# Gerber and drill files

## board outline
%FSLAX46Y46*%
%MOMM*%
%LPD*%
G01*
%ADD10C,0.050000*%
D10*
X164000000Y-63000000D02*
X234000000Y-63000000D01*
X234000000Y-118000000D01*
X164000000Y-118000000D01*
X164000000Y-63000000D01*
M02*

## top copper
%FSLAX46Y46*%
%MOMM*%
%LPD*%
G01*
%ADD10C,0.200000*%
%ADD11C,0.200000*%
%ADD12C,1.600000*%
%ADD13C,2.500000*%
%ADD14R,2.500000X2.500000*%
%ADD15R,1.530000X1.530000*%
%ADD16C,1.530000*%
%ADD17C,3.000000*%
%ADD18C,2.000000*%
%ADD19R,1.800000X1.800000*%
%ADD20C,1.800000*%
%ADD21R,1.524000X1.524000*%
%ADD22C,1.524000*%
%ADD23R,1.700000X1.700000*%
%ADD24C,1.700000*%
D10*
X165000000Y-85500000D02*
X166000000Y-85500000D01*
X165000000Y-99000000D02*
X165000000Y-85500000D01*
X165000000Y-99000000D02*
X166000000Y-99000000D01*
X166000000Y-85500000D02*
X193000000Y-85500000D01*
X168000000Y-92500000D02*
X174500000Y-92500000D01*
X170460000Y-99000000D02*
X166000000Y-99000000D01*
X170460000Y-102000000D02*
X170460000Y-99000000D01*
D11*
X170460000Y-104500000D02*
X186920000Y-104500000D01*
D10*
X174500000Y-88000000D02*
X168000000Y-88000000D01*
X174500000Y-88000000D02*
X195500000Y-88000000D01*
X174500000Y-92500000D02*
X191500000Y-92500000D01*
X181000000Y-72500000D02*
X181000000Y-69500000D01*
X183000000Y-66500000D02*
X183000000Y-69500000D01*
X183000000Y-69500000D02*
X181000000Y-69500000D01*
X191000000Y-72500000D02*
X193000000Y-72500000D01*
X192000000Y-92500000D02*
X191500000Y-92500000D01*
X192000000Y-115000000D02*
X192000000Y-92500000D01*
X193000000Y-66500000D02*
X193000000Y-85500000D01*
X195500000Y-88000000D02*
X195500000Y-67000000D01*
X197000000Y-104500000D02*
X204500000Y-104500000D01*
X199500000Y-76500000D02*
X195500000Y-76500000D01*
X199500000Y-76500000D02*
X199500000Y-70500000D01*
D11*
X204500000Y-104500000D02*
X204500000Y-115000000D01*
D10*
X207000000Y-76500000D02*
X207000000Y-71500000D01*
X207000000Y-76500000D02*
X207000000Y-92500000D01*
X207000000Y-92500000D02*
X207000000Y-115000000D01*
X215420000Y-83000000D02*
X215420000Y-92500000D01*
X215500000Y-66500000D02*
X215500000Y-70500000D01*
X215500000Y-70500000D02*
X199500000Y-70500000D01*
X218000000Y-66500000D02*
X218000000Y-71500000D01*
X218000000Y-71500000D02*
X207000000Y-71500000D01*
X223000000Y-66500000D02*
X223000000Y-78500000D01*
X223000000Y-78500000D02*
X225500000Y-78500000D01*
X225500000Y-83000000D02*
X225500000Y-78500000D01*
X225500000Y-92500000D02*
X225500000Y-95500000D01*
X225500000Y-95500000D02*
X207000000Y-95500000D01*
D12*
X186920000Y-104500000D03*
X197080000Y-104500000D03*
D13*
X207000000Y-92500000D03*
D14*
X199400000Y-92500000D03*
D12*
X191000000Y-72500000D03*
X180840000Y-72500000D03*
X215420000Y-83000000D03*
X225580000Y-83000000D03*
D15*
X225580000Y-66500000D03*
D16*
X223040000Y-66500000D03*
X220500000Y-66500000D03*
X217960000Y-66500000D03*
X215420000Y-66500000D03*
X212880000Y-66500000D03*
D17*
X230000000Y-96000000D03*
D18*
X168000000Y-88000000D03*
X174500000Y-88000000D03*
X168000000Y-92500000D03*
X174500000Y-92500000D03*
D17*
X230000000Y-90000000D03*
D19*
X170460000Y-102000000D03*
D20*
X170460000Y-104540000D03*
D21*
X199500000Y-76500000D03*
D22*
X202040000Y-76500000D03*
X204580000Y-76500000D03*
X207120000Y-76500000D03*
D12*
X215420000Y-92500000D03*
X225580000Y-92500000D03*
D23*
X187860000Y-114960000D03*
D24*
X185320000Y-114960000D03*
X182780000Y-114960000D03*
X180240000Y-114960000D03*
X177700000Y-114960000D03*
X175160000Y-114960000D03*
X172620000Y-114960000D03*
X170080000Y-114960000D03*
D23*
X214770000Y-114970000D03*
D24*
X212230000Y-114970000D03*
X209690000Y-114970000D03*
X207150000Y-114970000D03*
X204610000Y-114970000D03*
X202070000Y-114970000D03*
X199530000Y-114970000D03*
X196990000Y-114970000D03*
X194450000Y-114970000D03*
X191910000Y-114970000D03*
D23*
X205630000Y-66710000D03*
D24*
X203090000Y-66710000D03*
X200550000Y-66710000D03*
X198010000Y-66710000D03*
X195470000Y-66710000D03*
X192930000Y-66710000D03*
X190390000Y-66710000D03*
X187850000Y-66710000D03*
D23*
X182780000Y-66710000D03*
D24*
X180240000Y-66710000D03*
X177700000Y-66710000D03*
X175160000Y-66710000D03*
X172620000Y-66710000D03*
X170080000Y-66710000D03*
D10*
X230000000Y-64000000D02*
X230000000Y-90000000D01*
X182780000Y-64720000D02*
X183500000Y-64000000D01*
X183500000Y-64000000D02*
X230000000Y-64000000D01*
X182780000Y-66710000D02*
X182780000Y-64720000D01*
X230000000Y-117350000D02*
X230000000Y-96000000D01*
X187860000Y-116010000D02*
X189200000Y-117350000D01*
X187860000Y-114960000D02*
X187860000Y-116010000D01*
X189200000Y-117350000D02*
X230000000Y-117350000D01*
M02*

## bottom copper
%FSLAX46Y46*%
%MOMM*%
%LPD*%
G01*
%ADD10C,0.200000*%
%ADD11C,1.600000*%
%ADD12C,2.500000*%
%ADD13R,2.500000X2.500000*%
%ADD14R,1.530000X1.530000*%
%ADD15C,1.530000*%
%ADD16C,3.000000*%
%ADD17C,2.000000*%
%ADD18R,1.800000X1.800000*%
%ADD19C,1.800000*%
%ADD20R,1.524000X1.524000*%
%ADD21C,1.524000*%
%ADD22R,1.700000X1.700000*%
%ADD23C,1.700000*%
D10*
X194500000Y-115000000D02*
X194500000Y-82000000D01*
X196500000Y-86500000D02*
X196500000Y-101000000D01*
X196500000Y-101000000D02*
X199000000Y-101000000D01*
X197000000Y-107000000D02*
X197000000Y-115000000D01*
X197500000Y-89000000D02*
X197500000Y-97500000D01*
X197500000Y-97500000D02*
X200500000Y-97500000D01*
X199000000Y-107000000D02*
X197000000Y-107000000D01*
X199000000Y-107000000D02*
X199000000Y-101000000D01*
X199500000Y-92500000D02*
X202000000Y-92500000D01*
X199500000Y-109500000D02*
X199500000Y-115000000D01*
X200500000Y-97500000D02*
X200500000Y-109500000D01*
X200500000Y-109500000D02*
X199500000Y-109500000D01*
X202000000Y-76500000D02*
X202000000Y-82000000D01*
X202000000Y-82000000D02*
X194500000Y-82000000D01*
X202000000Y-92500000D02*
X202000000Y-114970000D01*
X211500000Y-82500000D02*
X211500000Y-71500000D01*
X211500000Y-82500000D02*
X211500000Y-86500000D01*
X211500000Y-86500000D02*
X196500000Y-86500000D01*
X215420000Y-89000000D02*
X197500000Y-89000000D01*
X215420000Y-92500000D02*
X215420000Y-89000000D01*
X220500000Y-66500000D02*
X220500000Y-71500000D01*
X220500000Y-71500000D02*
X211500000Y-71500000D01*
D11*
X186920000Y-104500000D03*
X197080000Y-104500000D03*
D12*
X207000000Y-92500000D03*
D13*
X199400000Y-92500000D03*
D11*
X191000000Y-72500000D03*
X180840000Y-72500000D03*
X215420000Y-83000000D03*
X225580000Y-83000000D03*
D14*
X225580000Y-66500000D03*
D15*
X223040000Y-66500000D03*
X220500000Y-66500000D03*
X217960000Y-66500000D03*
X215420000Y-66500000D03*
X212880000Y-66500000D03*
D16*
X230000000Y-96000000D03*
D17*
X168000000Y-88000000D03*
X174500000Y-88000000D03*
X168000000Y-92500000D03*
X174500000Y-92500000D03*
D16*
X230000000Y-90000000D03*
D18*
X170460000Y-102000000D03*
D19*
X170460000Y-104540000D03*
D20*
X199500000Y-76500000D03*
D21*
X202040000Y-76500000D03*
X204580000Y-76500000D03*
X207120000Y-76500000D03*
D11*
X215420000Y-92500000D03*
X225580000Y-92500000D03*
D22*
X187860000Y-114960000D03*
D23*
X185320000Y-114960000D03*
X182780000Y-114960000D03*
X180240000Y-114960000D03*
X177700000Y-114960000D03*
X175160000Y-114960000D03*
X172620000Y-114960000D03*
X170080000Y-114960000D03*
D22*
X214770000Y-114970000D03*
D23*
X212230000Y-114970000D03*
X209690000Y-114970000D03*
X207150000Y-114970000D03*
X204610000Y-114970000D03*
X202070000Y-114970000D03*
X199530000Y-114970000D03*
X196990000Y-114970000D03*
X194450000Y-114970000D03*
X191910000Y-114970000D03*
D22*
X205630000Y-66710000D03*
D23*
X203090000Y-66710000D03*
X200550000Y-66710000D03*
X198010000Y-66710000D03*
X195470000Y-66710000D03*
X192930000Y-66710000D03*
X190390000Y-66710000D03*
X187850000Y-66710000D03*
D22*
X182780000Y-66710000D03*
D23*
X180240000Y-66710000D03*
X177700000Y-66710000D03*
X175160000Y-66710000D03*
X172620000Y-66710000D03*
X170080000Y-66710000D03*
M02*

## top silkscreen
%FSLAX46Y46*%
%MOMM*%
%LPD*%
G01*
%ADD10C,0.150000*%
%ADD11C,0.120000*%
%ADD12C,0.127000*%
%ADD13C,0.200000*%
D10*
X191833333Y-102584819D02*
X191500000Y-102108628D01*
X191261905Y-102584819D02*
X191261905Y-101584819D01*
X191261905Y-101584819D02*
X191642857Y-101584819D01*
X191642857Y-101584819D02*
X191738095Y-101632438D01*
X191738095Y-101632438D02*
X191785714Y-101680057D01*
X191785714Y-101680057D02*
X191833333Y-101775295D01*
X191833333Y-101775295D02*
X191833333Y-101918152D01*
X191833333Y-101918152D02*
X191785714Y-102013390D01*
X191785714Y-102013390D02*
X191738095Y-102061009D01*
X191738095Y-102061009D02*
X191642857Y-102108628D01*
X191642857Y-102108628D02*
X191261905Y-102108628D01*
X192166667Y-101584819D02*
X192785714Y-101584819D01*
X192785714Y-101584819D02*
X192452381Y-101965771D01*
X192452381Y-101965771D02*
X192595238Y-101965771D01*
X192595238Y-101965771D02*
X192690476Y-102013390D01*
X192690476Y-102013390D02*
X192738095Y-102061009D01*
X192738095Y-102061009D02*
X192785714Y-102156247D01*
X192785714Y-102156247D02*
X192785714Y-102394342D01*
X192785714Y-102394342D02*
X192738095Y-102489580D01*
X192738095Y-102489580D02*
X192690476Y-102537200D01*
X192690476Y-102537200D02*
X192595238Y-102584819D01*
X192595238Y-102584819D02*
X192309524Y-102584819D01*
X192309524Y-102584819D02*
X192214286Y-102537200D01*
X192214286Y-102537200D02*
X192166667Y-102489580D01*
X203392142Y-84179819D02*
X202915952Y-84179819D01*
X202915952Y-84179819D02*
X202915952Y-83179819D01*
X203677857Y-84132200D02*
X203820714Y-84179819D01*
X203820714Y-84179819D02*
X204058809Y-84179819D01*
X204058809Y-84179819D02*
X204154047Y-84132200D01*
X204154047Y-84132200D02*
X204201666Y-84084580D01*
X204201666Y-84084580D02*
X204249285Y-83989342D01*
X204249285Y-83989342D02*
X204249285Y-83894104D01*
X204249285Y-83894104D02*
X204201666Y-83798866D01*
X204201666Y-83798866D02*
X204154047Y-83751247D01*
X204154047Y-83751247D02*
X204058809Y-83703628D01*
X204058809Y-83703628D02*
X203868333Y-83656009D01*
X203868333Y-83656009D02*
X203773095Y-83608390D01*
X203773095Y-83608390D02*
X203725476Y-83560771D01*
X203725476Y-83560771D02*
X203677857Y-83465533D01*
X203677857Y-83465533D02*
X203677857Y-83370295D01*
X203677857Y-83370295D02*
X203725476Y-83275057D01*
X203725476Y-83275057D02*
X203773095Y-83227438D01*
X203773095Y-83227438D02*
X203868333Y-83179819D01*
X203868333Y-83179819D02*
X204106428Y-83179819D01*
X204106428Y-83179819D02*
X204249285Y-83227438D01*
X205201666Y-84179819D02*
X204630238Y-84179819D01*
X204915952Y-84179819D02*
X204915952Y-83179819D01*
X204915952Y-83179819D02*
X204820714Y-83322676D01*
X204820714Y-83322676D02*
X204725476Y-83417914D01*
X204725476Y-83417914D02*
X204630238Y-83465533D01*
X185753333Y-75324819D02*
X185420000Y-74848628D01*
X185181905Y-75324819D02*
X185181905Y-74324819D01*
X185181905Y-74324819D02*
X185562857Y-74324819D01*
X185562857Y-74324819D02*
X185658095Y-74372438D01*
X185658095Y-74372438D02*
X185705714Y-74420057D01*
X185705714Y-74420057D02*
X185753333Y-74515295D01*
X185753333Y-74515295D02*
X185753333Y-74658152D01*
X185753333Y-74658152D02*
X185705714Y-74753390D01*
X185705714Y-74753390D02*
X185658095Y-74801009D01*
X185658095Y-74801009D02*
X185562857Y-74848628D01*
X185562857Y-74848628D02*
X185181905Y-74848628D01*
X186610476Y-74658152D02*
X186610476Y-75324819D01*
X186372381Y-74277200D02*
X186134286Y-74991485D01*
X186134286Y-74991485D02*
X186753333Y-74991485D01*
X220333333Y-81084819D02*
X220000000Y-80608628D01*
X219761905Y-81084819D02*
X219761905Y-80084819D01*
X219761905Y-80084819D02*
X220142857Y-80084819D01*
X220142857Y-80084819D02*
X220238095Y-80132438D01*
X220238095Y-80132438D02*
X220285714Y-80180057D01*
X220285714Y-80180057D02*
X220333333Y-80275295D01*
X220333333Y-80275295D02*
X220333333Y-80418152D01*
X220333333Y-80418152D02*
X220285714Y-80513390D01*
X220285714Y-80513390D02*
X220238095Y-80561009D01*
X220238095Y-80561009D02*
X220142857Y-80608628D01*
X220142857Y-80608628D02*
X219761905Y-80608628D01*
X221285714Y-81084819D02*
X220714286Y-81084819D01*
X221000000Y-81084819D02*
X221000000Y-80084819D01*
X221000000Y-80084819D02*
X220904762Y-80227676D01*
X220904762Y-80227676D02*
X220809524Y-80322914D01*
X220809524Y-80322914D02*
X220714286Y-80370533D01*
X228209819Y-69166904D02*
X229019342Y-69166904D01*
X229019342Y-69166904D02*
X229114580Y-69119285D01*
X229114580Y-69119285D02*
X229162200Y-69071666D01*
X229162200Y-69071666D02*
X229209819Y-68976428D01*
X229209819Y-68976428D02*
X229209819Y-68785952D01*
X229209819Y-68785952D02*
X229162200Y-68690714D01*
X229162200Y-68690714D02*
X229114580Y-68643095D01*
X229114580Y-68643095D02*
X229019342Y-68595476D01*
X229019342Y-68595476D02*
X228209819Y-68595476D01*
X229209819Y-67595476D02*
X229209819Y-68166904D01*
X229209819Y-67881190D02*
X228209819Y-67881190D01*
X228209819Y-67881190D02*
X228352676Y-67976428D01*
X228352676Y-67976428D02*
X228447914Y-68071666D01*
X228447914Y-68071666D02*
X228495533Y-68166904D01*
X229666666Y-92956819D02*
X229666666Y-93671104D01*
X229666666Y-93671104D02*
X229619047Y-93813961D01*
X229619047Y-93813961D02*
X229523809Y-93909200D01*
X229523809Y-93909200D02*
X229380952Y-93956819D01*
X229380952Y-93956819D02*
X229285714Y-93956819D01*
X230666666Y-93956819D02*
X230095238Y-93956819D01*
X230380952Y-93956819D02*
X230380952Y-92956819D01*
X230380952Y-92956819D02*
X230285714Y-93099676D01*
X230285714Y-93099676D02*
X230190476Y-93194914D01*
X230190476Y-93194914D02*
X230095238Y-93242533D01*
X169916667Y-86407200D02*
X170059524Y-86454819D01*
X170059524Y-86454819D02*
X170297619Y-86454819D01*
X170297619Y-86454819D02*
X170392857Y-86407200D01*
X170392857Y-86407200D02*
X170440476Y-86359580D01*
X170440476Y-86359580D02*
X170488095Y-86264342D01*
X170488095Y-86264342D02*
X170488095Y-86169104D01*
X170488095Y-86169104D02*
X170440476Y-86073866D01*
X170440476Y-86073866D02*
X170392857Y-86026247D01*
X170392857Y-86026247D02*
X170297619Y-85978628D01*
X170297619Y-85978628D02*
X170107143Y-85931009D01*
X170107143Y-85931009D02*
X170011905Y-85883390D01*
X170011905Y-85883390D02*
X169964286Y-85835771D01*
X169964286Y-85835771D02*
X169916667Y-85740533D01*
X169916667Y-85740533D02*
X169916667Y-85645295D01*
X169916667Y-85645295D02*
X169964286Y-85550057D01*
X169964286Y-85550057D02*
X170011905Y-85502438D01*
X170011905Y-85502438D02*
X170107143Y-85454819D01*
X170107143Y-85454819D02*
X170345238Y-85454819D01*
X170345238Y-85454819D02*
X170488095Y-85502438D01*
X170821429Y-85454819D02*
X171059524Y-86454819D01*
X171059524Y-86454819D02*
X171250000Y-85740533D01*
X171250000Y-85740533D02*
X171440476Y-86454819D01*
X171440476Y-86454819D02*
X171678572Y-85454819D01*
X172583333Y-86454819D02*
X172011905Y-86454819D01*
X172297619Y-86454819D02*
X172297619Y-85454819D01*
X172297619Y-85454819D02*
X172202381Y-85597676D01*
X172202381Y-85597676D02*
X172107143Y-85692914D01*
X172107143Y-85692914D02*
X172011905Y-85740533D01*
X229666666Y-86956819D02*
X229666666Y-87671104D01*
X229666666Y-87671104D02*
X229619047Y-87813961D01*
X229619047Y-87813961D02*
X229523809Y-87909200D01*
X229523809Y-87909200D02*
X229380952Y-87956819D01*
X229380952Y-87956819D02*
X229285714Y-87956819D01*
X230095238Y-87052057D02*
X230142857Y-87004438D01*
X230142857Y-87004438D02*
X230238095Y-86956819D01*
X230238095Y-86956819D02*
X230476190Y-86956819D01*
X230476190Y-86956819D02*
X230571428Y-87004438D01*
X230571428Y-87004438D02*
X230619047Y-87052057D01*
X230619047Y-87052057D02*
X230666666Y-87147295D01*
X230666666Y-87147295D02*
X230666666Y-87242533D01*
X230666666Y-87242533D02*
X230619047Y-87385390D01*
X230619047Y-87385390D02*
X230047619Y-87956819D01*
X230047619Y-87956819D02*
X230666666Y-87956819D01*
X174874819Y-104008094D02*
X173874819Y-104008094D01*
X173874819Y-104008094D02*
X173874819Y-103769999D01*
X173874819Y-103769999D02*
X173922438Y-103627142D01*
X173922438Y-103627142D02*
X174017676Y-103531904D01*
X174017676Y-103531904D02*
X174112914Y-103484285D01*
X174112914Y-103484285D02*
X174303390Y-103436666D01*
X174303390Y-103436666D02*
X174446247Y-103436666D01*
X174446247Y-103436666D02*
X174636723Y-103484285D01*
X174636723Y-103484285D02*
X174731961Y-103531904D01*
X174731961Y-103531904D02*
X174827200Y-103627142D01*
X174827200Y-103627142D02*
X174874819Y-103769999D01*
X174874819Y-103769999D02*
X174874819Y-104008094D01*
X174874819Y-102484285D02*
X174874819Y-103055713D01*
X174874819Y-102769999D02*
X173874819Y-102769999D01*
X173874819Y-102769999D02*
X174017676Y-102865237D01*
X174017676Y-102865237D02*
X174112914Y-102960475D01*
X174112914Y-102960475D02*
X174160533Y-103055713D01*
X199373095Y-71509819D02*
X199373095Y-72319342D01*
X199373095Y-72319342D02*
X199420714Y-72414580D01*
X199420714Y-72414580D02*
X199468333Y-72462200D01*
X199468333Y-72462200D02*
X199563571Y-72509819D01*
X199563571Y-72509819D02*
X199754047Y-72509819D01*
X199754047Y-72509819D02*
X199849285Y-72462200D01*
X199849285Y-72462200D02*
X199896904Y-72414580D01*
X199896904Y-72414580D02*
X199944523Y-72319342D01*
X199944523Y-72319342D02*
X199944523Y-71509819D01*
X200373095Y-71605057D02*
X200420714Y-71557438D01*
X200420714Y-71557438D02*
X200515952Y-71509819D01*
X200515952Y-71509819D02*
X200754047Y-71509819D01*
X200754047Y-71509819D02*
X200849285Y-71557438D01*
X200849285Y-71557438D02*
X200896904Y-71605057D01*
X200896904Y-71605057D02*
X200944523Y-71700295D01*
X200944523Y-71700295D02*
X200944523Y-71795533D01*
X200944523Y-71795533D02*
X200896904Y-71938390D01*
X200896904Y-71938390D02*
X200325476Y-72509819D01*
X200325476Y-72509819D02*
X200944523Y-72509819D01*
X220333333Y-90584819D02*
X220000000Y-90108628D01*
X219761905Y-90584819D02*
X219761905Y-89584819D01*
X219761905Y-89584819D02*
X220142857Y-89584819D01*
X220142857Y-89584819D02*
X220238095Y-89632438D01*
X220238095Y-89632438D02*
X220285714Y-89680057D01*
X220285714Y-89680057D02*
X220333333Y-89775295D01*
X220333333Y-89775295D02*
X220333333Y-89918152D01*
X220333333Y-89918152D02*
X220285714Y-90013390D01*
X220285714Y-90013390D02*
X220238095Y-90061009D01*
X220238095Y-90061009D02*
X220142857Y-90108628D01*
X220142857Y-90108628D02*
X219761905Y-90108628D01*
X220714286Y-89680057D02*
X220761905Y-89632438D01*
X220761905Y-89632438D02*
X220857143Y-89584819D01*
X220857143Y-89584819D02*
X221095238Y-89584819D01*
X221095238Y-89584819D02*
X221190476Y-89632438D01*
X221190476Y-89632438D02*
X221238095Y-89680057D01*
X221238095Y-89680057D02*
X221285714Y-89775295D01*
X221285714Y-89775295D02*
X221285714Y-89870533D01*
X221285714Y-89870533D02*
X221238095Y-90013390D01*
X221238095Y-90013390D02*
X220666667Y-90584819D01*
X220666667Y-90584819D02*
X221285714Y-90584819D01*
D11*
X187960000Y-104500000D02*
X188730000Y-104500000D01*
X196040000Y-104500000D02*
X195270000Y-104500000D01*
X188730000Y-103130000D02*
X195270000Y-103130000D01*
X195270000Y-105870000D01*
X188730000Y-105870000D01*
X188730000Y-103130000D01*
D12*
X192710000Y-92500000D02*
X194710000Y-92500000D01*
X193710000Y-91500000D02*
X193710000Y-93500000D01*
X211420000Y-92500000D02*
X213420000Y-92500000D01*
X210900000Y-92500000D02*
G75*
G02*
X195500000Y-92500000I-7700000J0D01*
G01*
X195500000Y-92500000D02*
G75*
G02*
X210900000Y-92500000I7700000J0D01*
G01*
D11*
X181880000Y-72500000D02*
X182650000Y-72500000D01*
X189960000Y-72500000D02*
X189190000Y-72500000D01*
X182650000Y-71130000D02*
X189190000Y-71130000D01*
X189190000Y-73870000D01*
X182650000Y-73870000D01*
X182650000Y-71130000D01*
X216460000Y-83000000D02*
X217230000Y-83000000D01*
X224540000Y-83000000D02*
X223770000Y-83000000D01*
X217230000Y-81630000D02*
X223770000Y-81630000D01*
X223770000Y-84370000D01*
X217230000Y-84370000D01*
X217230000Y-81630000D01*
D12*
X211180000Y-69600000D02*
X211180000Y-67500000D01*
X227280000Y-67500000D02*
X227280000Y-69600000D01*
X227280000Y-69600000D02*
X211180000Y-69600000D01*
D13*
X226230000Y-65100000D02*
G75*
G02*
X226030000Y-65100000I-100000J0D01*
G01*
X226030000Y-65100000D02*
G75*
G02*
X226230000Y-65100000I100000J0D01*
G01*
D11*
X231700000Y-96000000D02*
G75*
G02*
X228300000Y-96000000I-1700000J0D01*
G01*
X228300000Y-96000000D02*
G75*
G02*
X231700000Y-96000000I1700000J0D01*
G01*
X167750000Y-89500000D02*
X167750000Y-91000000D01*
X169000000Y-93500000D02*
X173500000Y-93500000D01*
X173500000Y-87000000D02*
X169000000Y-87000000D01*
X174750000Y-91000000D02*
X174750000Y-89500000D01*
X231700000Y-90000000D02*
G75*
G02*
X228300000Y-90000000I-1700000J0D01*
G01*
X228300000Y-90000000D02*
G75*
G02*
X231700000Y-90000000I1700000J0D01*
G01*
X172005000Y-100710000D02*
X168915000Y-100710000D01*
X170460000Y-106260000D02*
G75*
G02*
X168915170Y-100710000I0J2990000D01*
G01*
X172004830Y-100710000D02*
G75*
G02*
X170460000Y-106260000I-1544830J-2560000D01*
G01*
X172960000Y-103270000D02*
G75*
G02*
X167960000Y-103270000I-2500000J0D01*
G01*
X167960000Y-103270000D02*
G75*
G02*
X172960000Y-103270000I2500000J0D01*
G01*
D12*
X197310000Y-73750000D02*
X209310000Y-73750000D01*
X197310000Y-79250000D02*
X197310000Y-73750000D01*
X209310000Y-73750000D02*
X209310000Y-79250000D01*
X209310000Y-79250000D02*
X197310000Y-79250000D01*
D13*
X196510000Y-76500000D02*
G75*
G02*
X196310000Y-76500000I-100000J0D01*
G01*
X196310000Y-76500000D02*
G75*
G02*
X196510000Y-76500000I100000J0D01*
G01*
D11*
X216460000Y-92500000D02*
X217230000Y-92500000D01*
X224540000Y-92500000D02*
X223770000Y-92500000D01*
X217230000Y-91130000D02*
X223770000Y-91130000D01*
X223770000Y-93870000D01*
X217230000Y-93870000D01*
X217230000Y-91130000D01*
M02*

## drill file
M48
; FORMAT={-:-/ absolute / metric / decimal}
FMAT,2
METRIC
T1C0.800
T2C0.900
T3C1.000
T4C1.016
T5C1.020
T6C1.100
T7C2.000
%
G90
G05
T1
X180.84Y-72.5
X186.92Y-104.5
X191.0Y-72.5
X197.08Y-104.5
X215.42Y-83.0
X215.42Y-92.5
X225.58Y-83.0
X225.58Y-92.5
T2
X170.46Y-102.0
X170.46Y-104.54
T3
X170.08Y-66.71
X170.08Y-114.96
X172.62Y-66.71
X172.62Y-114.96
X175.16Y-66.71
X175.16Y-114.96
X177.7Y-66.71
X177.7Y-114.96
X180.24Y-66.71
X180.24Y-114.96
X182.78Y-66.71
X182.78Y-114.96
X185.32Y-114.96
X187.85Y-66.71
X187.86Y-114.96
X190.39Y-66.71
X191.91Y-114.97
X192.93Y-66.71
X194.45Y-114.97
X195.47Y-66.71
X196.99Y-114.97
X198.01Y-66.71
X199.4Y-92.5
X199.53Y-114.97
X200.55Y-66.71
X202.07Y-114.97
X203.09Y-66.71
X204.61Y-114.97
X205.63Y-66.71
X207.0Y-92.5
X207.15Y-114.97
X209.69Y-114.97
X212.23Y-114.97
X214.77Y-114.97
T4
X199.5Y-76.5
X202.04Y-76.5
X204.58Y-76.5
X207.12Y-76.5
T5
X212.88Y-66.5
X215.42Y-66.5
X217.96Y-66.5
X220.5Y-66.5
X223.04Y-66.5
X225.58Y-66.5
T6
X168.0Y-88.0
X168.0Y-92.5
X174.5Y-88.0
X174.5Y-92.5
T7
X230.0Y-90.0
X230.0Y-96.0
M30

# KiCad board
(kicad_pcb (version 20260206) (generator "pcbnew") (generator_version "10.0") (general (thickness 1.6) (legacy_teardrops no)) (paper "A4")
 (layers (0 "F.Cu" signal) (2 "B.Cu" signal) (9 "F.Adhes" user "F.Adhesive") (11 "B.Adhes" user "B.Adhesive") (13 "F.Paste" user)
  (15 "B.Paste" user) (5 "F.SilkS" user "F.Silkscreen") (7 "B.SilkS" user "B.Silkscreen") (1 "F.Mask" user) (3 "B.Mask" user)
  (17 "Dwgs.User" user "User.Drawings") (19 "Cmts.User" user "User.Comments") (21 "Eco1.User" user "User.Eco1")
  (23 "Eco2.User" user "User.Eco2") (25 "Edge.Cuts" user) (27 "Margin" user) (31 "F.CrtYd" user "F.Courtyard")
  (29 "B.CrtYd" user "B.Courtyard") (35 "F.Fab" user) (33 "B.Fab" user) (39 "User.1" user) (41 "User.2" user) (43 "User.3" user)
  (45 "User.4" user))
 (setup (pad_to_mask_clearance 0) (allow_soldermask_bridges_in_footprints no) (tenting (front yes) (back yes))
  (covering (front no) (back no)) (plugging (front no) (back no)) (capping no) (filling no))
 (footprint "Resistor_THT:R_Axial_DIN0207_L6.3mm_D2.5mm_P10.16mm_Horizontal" (layer "F.Cu") (at 186.92 104.5)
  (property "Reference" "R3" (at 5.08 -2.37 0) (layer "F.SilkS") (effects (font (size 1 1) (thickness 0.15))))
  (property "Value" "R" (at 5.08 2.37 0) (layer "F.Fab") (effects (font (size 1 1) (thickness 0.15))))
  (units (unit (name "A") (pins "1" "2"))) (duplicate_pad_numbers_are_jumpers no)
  (fp_line (start 1.04 0) (end 1.81 0) (stroke (width 0.12) (type solid)) (layer "F.SilkS"))
  (fp_line (start 9.12 0) (end 8.35 0) (stroke (width 0.12) (type solid)) (layer "F.SilkS"))
  (fp_rect (start 1.81 -1.37) (end 8.35 1.37) (stroke (width 0.12) (type solid)) (fill no) (layer "F.SilkS"))
  (pad "1" thru_hole circle (at 0 0) (size 1.6 1.6) (drill 0.8) (layers "*.Cu" "*.Mask") (remove_unused_layers no) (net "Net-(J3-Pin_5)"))
  (pad "2" thru_hole circle (at 10.16 0) (size 1.6 1.6) (drill 0.8) (layers "*.Cu" "*.Mask") (remove_unused_layers no) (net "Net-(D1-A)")))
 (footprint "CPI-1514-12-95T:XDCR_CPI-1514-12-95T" (layer "F.Cu") (at 203.2 92.5)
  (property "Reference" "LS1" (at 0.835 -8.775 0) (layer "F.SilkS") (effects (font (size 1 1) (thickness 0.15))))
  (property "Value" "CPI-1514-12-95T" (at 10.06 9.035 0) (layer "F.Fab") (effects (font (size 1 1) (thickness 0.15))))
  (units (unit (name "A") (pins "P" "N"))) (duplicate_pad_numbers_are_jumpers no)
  (fp_line (start -10.49 0) (end -8.49 0) (stroke (width 0.127) (type solid)) (layer "F.SilkS"))
  (fp_line (start -9.49 -1) (end -9.49 1) (stroke (width 0.127) (type solid)) (layer "F.SilkS"))
  (fp_line (start 8.22 0) (end 10.22 0) (stroke (width 0.127) (type solid)) (layer "F.SilkS"))
  (fp_circle (center 0 0) (end 7.7 0) (stroke (width 0.127) (type solid)) (fill no) (layer "F.SilkS"))
  (pad "N" thru_hole circle (at 3.8 0) (size 2.5 2.5) (drill 1) (layers "*.Cu" "*.Mask") (remove_unused_layers no) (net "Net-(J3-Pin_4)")
   (solder_mask_margin 0.102))
  (pad "P" thru_hole rect (at -3.8 0) (size 2.5 2.5) (drill 1) (layers "*.Cu" "*.Mask") (remove_unused_layers no) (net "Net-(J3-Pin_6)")
   (solder_mask_margin 0.102)))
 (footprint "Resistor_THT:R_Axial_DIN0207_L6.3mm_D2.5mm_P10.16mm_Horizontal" (layer "F.Cu") (at 191 72.5 180)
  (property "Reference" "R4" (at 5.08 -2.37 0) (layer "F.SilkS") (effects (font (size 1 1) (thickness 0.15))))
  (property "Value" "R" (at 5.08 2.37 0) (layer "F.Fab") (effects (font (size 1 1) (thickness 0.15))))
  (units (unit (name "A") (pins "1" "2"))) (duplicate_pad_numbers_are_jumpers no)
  (fp_line (start 9.12 0) (end 8.35 0) (stroke (width 0.12) (type solid)) (layer "F.SilkS"))
  (fp_line (start 1.04 0) (end 1.81 0) (stroke (width 0.12) (type solid)) (layer "F.SilkS"))
  (fp_rect (start 1.81 -1.37) (end 8.35 1.37) (stroke (width 0.12) (type solid)) (fill no) (layer "F.SilkS"))
  (pad "1" thru_hole circle (at 0 0 180) (size 1.6 1.6) (drill 0.8) (layers "*.Cu" "*.Mask") (remove_unused_layers no) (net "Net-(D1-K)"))
  (pad "2" thru_hole circle (at 10.16 0 180) (size 1.6 1.6) (drill 0.8) (layers "*.Cu" "*.Mask") (remove_unused_layers no)
   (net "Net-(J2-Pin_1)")))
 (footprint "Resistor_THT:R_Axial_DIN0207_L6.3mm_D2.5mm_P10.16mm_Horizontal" (layer "F.Cu") (at 215.42 83)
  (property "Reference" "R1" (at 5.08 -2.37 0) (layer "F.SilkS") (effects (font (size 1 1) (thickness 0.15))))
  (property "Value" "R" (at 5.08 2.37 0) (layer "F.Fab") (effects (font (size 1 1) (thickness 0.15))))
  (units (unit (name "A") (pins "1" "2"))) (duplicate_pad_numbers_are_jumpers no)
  (fp_line (start 1.04 0) (end 1.81 0) (stroke (width 0.12) (type solid)) (layer "F.SilkS"))
  (fp_line (start 9.12 0) (end 8.35 0) (stroke (width 0.12) (type solid)) (layer "F.SilkS"))
  (fp_rect (start 1.81 -1.37) (end 8.35 1.37) (stroke (width 0.12) (type solid)) (fill no) (layer "F.SilkS"))
  (pad "1" thru_hole circle (at 0 0) (size 1.6 1.6) (drill 0.8) (layers "*.Cu" "*.Mask") (remove_unused_layers no) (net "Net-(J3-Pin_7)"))
  (pad "2" thru_hole circle (at 10.16 0) (size 1.6 1.6) (drill 0.8) (layers "*.Cu" "*.Mask") (remove_unused_layers no) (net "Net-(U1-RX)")))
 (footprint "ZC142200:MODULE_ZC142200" (layer "F.Cu") (at 219.23 66.5 -90)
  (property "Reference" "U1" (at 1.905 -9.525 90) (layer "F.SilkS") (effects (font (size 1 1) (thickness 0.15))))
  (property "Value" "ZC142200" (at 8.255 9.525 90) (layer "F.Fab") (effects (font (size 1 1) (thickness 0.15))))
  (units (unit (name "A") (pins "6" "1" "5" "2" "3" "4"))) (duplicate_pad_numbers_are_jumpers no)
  (fp_line (start 3.1 8.05) (end 1 8.05) (stroke (width 0.127) (type solid)) (layer "F.SilkS"))
  (fp_line (start 1 -8.05) (end 3.1 -8.05) (stroke (width 0.127) (type solid)) (layer "F.SilkS"))
  (fp_line (start 3.1 -8.05) (end 3.1 8.05) (stroke (width 0.127) (type solid)) (layer "F.SilkS"))
  (fp_circle (center -1.4 -6.9) (end -1.3 -6.9) (stroke (width 0.2) (type solid)) (fill no) (layer "F.SilkS"))
  (pad "1" thru_hole rect (at 0 -6.35 270) (size 1.53 1.53) (drill 1.02) (layers "*.Cu" "*.Mask") (remove_unused_layers no)
   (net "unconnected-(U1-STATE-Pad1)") (solder_mask_margin 0.102))
  (pad "2" thru_hole circle (at 0 -3.81 270) (size 1.53 1.53) (drill 1.02) (layers "*.Cu" "*.Mask") (remove_unused_layers no)
   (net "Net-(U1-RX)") (solder_mask_margin 0.102))
  (pad "3" thru_hole circle (at 0 -1.27 270) (size 1.53 1.53) (drill 1.02) (layers "*.Cu" "*.Mask") (remove_unused_layers no)
   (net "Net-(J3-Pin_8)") (solder_mask_margin 0.102))
  (pad "4" thru_hole circle (at 0 1.27 270) (size 1.53 1.53) (drill 1.02) (layers "*.Cu" "*.Mask") (remove_unused_layers no)
   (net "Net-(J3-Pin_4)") (solder_mask_margin 0.102))
  (pad "5" thru_hole circle (at 0 3.81 270) (size 1.53 1.53) (drill 1.02) (layers "*.Cu" "*.Mask") (remove_unused_layers no)
   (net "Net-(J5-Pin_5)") (solder_mask_margin 0.102))
  (pad "6" thru_hole circle (at 0 6.35 270) (size 1.53 1.53) (drill 1.02) (layers "*.Cu" "*.Mask") (remove_unused_layers no)
   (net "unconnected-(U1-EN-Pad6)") (solder_mask_margin 0.102)))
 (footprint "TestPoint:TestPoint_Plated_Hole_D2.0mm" (layer "F.Cu") (at 230 96)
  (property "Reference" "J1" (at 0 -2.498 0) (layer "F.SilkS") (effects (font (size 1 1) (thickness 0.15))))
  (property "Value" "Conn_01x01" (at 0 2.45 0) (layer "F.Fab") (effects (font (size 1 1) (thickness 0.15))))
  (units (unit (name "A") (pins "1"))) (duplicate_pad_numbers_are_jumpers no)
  (fp_circle (center 0 0) (end 0 -1.7) (stroke (width 0.12) (type solid)) (fill no) (layer "F.SilkS"))
  (pad "1" thru_hole circle (at 0 0) (size 3 3) (drill 2) (layers "*.Cu" "*.Mask") (remove_unused_layers no) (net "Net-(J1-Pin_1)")))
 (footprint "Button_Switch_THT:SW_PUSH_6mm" (layer "F.Cu") (at 168 88)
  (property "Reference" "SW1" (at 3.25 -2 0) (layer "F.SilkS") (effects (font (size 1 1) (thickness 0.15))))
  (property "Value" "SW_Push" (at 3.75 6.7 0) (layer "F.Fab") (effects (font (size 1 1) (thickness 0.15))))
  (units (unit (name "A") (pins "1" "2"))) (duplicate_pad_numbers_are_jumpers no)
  (fp_line (start -0.25 1.5) (end -0.25 3) (stroke (width 0.12) (type solid)) (layer "F.SilkS"))
  (fp_line (start 1 5.5) (end 5.5 5.5) (stroke (width 0.12) (type solid)) (layer "F.SilkS"))
  (fp_line (start 5.5 -1) (end 1 -1) (stroke (width 0.12) (type solid)) (layer "F.SilkS"))
  (fp_line (start 6.75 3) (end 6.75 1.5) (stroke (width 0.12) (type solid)) (layer "F.SilkS"))
  (pad "1" thru_hole circle (at 0 0 90) (size 2 2) (drill 1.1) (layers "*.Cu" "*.Mask") (remove_unused_layers no) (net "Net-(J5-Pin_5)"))
  (pad "1" thru_hole circle (at 6.5 0 90) (size 2 2) (drill 1.1) (layers "*.Cu" "*.Mask") (remove_unused_layers no) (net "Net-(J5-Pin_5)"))
  (pad "2" thru_hole circle (at 0 4.5 90) (size 2 2) (drill 1.1) (layers "*.Cu" "*.Mask") (remove_unused_layers no) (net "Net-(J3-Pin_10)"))
  (pad "2" thru_hole circle (at 6.5 4.5 90) (size 2 2) (drill 1.1) (layers "*.Cu" "*.Mask") (remove_unused_layers no)
   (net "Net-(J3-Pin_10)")))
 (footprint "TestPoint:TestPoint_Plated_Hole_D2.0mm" (layer "F.Cu") (at 230 90)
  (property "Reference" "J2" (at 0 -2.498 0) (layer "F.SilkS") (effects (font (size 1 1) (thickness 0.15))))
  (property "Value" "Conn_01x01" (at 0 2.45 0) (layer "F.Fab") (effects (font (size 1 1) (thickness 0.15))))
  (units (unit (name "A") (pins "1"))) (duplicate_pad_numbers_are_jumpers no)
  (fp_circle (center 0 0) (end 0 -1.7) (stroke (width 0.12) (type solid)) (fill no) (layer "F.SilkS"))
  (pad "1" thru_hole circle (at 0 0) (size 3 3) (drill 2) (layers "*.Cu" "*.Mask") (remove_unused_layers no) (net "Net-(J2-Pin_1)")))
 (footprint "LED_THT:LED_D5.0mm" (layer "F.Cu") (at 170.46 102 -90)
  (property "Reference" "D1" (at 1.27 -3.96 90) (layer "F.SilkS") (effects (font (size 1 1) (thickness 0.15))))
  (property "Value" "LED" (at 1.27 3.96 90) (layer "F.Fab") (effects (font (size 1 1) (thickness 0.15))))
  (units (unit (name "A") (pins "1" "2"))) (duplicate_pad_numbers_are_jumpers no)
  (fp_line (start -1.29 -1.545) (end -1.29 1.545) (stroke (width 0.12) (type solid)) (layer "F.SilkS"))
  (fp_arc (start 4.26 0) (mid 2.071779 2.880495) (end -1.29 1.54483) (stroke (width 0.12) (type solid)) (layer "F.SilkS"))
  (fp_arc (start -1.29 -1.54483) (mid 2.071779 -2.880495) (end 4.26 0) (stroke (width 0.12) (type solid)) (layer "F.SilkS"))
  (fp_circle (center 1.27 0) (end 3.77 0) (stroke (width 0.12) (type solid)) (fill no) (layer "F.SilkS"))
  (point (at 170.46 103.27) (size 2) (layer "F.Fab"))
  (pad "1" thru_hole rect (at 0 0 270) (size 1.8 1.8) (drill 0.9) (layers "*.Cu" "*.Mask") (remove_unused_layers no) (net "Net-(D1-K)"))
  (pad "2" thru_hole circle (at 2.54 0 270) (size 1.8 1.8) (drill 0.9) (layers "*.Cu" "*.Mask") (remove_unused_layers no) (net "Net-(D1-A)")))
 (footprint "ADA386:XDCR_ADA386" (layer "F.Cu") (at 203.31 76.5)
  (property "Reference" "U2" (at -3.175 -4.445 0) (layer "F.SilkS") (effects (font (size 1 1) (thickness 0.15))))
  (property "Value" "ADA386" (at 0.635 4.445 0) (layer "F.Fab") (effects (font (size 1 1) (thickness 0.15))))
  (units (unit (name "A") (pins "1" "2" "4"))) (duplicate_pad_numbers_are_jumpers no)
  (fp_line (start -6 -2.75) (end 6 -2.75) (stroke (width 0.127) (type solid)) (layer "F.SilkS"))
  (fp_line (start -6 2.75) (end -6 -2.75) (stroke (width 0.127) (type solid)) (layer "F.SilkS"))
  (fp_line (start 6 -2.75) (end 6 2.75) (stroke (width 0.127) (type solid)) (layer "F.SilkS"))
  (fp_line (start 6 2.75) (end -6 2.75) (stroke (width 0.127) (type solid)) (layer "F.SilkS"))
  (fp_circle (center -6.9 0) (end -6.8 0) (stroke (width 0.2) (type solid)) (fill no) (layer "F.SilkS"))
  (pad "1" thru_hole rect (at -3.81 0) (size 1.524 1.524) (drill 1.016) (layers "*.Cu" "*.Mask") (remove_unused_layers no)
   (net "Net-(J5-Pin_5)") (solder_mask_margin 0.102))
  (pad "2" thru_hole circle (at -1.27 0) (size 1.524 1.524) (drill 1.016) (layers "*.Cu" "*.Mask") (remove_unused_layers no)
   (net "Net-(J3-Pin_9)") (solder_mask_margin 0.102))
  (pad "3" thru_hole circle (at 1.27 0) (size 1.524 1.524) (drill 1.016) (layers "*.Cu" "*.Mask") (remove_unused_layers no)
   (solder_mask_margin 0.102))
  (pad "4" thru_hole circle (at 3.81 0) (size 1.524 1.524) (drill 1.016) (layers "*.Cu" "*.Mask") (remove_unused_layers no)
   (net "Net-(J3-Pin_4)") (solder_mask_margin 0.102)))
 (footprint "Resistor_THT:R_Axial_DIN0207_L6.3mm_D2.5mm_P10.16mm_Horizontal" (layer "F.Cu") (at 215.42 92.5)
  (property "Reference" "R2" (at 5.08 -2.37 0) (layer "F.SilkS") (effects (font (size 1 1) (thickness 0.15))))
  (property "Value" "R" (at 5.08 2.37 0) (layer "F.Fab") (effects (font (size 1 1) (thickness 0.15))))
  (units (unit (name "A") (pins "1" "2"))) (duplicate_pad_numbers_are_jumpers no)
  (fp_line (start 1.04 0) (end 1.81 0) (stroke (width 0.12) (type solid)) (layer "F.SilkS"))
  (fp_line (start 9.12 0) (end 8.35 0) (stroke (width 0.12) (type solid)) (layer "F.SilkS"))
  (fp_rect (start 1.81 -1.37) (end 8.35 1.37) (stroke (width 0.12) (type solid)) (fill no) (layer "F.SilkS"))
  (pad "1" thru_hole circle (at 0 0) (size 1.6 1.6) (drill 0.8) (layers "*.Cu" "*.Mask") (remove_unused_layers no) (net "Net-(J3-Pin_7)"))
  (pad "2" thru_hole circle (at 10.16 0) (size 1.6 1.6) (drill 0.8) (layers "*.Cu" "*.Mask") (remove_unused_layers no)
   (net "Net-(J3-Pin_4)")))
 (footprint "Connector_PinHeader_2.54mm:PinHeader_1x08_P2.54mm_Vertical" (layer "B.Cu") (at 187.86 114.96 90)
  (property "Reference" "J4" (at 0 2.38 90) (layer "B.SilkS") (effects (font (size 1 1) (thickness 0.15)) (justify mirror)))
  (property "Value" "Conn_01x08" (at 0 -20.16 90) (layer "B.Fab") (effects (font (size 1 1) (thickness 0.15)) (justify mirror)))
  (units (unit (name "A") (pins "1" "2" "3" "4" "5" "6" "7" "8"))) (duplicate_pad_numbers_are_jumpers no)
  (pad "1" thru_hole rect (at 0 0 90) (size 1.7 1.7) (drill 1) (layers "*.Cu" "*.Mask") (remove_unused_layers no) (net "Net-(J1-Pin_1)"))
  (pad "2" thru_hole circle (at 0 -2.54 90) (size 1.7 1.7) (drill 1) (layers "*.Cu" "*.Mask") (remove_unused_layers no)
   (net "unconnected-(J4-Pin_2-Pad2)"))
  (pad "3" thru_hole circle (at 0 -5.08 90) (size 1.7 1.7) (drill 1) (layers "*.Cu" "*.Mask") (remove_unused_layers no)
   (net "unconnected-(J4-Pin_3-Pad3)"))
  (pad "4" thru_hole circle (at 0 -7.62 90) (size 1.7 1.7) (drill 1) (layers "*.Cu" "*.Mask") (remove_unused_layers no)
   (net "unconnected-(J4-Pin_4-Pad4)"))
  (pad "5" thru_hole circle (at 0 -10.16 90) (size 1.7 1.7) (drill 1) (layers "*.Cu" "*.Mask") (remove_unused_layers no)
   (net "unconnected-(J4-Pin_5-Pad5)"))
  (pad "6" thru_hole circle (at 0 -12.7 90) (size 1.7 1.7) (drill 1) (layers "*.Cu" "*.Mask") (remove_unused_layers no)
   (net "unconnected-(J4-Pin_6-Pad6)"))
  (pad "7" thru_hole circle (at 0 -15.24 90) (size 1.7 1.7) (drill 1) (layers "*.Cu" "*.Mask") (remove_unused_layers no)
   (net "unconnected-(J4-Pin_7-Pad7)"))
  (pad "8" thru_hole circle (at 0 -17.78 90) (size 1.7 1.7) (drill 1) (layers "*.Cu" "*.Mask") (remove_unused_layers no)
   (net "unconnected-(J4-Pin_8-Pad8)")))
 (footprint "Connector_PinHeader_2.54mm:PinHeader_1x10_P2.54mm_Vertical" (layer "B.Cu") (at 214.77 114.97 90)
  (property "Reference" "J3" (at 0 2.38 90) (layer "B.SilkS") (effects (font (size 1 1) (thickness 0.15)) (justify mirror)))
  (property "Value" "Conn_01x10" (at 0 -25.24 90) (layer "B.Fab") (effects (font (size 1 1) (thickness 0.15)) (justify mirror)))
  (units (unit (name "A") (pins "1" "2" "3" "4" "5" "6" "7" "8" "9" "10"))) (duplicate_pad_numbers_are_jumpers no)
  (pad "1" thru_hole rect (at 0 0 90) (size 1.7 1.7) (drill 1) (layers "*.Cu" "*.Mask") (remove_unused_layers no)
   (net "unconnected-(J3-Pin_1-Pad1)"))
  (pad "2" thru_hole circle (at 0 -2.54 90) (size 1.7 1.7) (drill 1) (layers "*.Cu" "*.Mask") (remove_unused_layers no)
   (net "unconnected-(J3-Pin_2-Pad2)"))
  (pad "3" thru_hole circle (at 0 -5.08 90) (size 1.7 1.7) (drill 1) (layers "*.Cu" "*.Mask") (remove_unused_layers no)
   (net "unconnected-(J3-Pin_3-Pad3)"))
  (pad "4" thru_hole circle (at 0 -7.62 90) (size 1.7 1.7) (drill 1) (layers "*.Cu" "*.Mask") (remove_unused_layers no)
   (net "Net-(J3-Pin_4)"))
  (pad "5" thru_hole circle (at 0 -10.16 90) (size 1.7 1.7) (drill 1) (layers "*.Cu" "*.Mask") (remove_unused_layers no)
   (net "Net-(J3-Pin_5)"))
  (pad "6" thru_hole circle (at 0 -12.7 90) (size 1.7 1.7) (drill 1) (layers "*.Cu" "*.Mask") (remove_unused_layers no)
   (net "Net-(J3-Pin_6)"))
  (pad "7" thru_hole circle (at 0 -15.24 90) (size 1.7 1.7) (drill 1) (layers "*.Cu" "*.Mask") (remove_unused_layers no)
   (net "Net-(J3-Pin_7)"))
  (pad "8" thru_hole circle (at 0 -17.78 90) (size 1.7 1.7) (drill 1) (layers "*.Cu" "*.Mask") (remove_unused_layers no)
   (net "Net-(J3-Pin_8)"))
  (pad "9" thru_hole circle (at 0 -20.32 90) (size 1.7 1.7) (drill 1) (layers "*.Cu" "*.Mask") (remove_unused_layers no)
   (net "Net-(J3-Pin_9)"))
  (pad "10" thru_hole circle (at 0 -22.86 90) (size 1.7 1.7) (drill 1) (layers "*.Cu" "*.Mask") (remove_unused_layers no)
   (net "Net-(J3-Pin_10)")))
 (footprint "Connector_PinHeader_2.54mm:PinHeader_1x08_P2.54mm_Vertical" (layer "B.Cu") (at 205.63 66.71 90)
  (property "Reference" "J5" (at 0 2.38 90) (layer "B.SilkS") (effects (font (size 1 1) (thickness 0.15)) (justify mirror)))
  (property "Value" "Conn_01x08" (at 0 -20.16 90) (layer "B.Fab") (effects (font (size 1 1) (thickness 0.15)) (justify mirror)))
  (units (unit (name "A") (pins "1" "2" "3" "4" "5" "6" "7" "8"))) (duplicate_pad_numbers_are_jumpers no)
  (pad "1" thru_hole rect (at 0 0 90) (size 1.7 1.7) (drill 1) (layers "*.Cu" "*.Mask") (remove_unused_layers no)
   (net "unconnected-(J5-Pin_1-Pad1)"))
  (pad "2" thru_hole circle (at 0 -2.54 90) (size 1.7 1.7) (drill 1) (layers "*.Cu" "*.Mask") (remove_unused_layers no)
   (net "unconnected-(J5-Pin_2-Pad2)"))
  (pad "3" thru_hole circle (at 0 -5.08 90) (size 1.7 1.7) (drill 1) (layers "*.Cu" "*.Mask") (remove_unused_layers no)
   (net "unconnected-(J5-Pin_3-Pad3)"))
  (pad "4" thru_hole circle (at 0 -7.62 90) (size 1.7 1.7) (drill 1) (layers "*.Cu" "*.Mask") (remove_unused_layers no)
   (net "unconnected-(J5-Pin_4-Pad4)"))
  (pad "5" thru_hole circle (at 0 -10.16 90) (size 1.7 1.7) (drill 1) (layers "*.Cu" "*.Mask") (remove_unused_layers no)
   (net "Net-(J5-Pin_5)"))
  (pad "6" thru_hole circle (at 0 -12.7 90) (size 1.7 1.7) (drill 1) (layers "*.Cu" "*.Mask") (remove_unused_layers no) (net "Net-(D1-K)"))
  (pad "7" thru_hole circle (at 0 -15.24 90) (size 1.7 1.7) (drill 1) (layers "*.Cu" "*.Mask") (remove_unused_layers no)
   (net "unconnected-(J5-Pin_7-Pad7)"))
  (pad "8" thru_hole circle (at 0 -17.78 90) (size 1.7 1.7) (drill 1) (layers "*.Cu" "*.Mask") (remove_unused_layers no)
   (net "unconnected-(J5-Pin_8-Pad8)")))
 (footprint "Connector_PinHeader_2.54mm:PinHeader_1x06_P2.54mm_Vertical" (layer "B.Cu") (at 182.78 66.71 90)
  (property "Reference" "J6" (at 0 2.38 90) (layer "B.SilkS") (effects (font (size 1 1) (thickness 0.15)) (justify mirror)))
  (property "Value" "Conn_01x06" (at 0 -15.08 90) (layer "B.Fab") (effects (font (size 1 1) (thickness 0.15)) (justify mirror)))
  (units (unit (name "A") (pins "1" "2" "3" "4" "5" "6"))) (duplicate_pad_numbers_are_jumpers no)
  (pad "1" thru_hole rect (at 0 0 90) (size 1.7 1.7) (drill 1) (layers "*.Cu" "*.Mask") (remove_unused_layers no) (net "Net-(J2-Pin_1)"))
  (pad "2" thru_hole circle (at 0 -2.54 90) (size 1.7 1.7) (drill 1) (layers "*.Cu" "*.Mask") (remove_unused_layers no)
   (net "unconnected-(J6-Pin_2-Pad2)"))
  (pad "3" thru_hole circle (at 0 -5.08 90) (size 1.7 1.7) (drill 1) (layers "*.Cu" "*.Mask") (remove_unused_layers no)
   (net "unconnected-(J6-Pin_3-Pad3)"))
  (pad "4" thru_hole circle (at 0 -7.62 90) (size 1.7 1.7) (drill 1) (layers "*.Cu" "*.Mask") (remove_unused_layers no)
   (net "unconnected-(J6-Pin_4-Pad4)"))
  (pad "5" thru_hole circle (at 0 -10.16 90) (size 1.7 1.7) (drill 1) (layers "*.Cu" "*.Mask") (remove_unused_layers no)
   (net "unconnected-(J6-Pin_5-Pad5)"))
  (pad "6" thru_hole circle (at 0 -12.7 90) (size 1.7 1.7) (drill 1) (layers "*.Cu" "*.Mask") (remove_unused_layers no)
   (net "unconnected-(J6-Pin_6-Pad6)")))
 (gr_line (start 165 85.5) (end 166 85.5) (stroke (width 0.2) (type default)) (layer "F.Cu") (net "Net-(D1-K)"))
 (gr_line (start 165 99) (end 165 85.5) (stroke (width 0.2) (type default)) (layer "F.Cu") (net "Net-(D1-K)"))
 (gr_line (start 165 99) (end 166 99) (stroke (width 0.2) (type default)) (layer "F.Cu") (net "Net-(D1-K)"))
 (gr_line (start 166 85.5) (end 193 85.5) (stroke (width 0.2) (type default)) (layer "F.Cu") (net "Net-(D1-K)"))
 (gr_line (start 168 92.5) (end 174.5 92.5) (stroke (width 0.2) (type default)) (layer "F.Cu") (net "Net-(J3-Pin_10)"))
 (gr_line (start 170.46 99) (end 166 99) (stroke (width 0.2) (type default)) (layer "F.Cu") (net "Net-(D1-K)"))
 (gr_line (start 170.46 102) (end 170.46 99) (stroke (width 0.2) (type default)) (layer "F.Cu") (net "Net-(D1-K)"))
 (gr_line (start 170.46 104.5) (end 186.92 104.5) (stroke (width 0.2) (type default)) (layer "F.Cu"))
 (gr_line (start 174.5 88) (end 168 88) (stroke (width 0.2) (type default)) (layer "F.Cu") (net "Net-(J5-Pin_5)"))
 (gr_line (start 174.5 88) (end 195.5 88) (stroke (width 0.2) (type default)) (layer "F.Cu") (net "Net-(J5-Pin_5)"))
 (gr_line (start 174.5 92.5) (end 191.5 92.5) (stroke (width 0.2) (type default)) (layer "F.Cu") (net "Net-(J3-Pin_10)"))
 (gr_line (start 181 72.5) (end 181 69.5) (stroke (width 0.2) (type default)) (layer "F.Cu") (net "Net-(J2-Pin_1)"))
 (gr_line (start 183 66.5) (end 183 69.5) (stroke (width 0.2) (type default)) (layer "F.Cu") (net "Net-(J2-Pin_1)"))
 (gr_line (start 183 69.5) (end 181 69.5) (stroke (width 0.2) (type default)) (layer "F.Cu") (net "Net-(J2-Pin_1)"))
 (gr_line (start 191 72.5) (end 193 72.5) (stroke (width 0.2) (type default)) (layer "F.Cu") (net "Net-(D1-K)"))
 (gr_line (start 192 92.5) (end 191.5 92.5) (stroke (width 0.2) (type default)) (layer "F.Cu") (net "Net-(J3-Pin_10)"))
 (gr_line (start 192 115) (end 192 92.5) (stroke (width 0.2) (type default)) (layer "F.Cu") (net "Net-(J3-Pin_10)"))
 (gr_line (start 193 66.5) (end 193 85.5) (stroke (width 0.2) (type default)) (layer "F.Cu") (net "Net-(D1-K)"))
 (gr_line (start 195.5 88) (end 195.5 67) (stroke (width 0.2) (type default)) (layer "F.Cu") (net "Net-(J5-Pin_5)"))
 (gr_line (start 197 104.5) (end 204.5 104.5) (stroke (width 0.2) (type default)) (layer "F.Cu") (net "Net-(D1-A)"))
 (gr_line (start 199.5 76.5) (end 195.5 76.5) (stroke (width 0.2) (type default)) (layer "F.Cu") (net "Net-(J5-Pin_5)"))
 (gr_line (start 199.5 76.5) (end 199.5 70.5) (stroke (width 0.2) (type default)) (layer "F.Cu") (net "Net-(J5-Pin_5)"))
 (gr_line (start 204.5 104.5) (end 204.5 115) (stroke (width 0.2) (type default)) (layer "F.Cu"))
 (gr_line (start 207 76.5) (end 207 71.5) (stroke (width 0.2) (type default)) (layer "F.Cu") (net "Net-(J3-Pin_4)"))
 (gr_line (start 207 76.5) (end 207 92.5) (stroke (width 0.2) (type default)) (layer "F.Cu") (net "Net-(J3-Pin_4)"))
 (gr_line (start 207 92.5) (end 207 115) (stroke (width 0.2) (type default)) (layer "F.Cu") (net "Net-(J3-Pin_4)"))
 (gr_line (start 215.42 83) (end 215.42 92.5) (stroke (width 0.2) (type default)) (layer "F.Cu") (net "Net-(J3-Pin_7)"))
 (gr_line (start 215.5 66.5) (end 215.5 70.5) (stroke (width 0.2) (type default)) (layer "F.Cu") (net "Net-(J5-Pin_5)"))
 (gr_line (start 215.5 70.5) (end 199.5 70.5) (stroke (width 0.2) (type default)) (layer "F.Cu") (net "Net-(J5-Pin_5)"))
 (gr_line (start 218 66.5) (end 218 71.5) (stroke (width 0.2) (type default)) (layer "F.Cu") (net "Net-(J3-Pin_4)"))
 (gr_line (start 218 71.5) (end 207 71.5) (stroke (width 0.2) (type default)) (layer "F.Cu") (net "Net-(J3-Pin_4)"))
 (gr_line (start 223 66.5) (end 223 78.5) (stroke (width 0.2) (type default)) (layer "F.Cu") (net "Net-(U1-RX)"))
 (gr_line (start 223 78.5) (end 225.5 78.5) (stroke (width 0.2) (type default)) (layer "F.Cu") (net "Net-(U1-RX)"))
 (gr_line (start 225.5 83) (end 225.5 78.5) (stroke (width 0.2) (type default)) (layer "F.Cu") (net "Net-(U1-RX)"))
 (gr_line (start 225.5 92.5) (end 225.5 95.5) (stroke (width 0.2) (type default)) (layer "F.Cu") (net "Net-(J3-Pin_4)"))
 (gr_line (start 225.5 95.5) (end 207 95.5) (stroke (width 0.2) (type default)) (layer "F.Cu") (net "Net-(J3-Pin_4)"))
 (gr_line (start 194.5 115) (end 194.5 82) (stroke (width 0.2) (type default)) (layer "B.Cu") (net "Net-(J3-Pin_9)"))
 (gr_line (start 196.5 86.5) (end 196.5 101) (stroke (width 0.2) (type default)) (layer "B.Cu") (net "Net-(J3-Pin_8)"))
 (gr_line (start 196.5 101) (end 199 101) (stroke (width 0.2) (type default)) (layer "B.Cu") (net "Net-(J3-Pin_8)"))
 (gr_line (start 197 107) (end 197 115) (stroke (width 0.2) (type default)) (layer "B.Cu") (net "Net-(J3-Pin_8)"))
 (gr_line (start 197.5 89) (end 197.5 97.5) (stroke (width 0.2) (type default)) (layer "B.Cu") (net "Net-(J3-Pin_7)"))
 (gr_line (start 197.5 97.5) (end 200.5 97.5) (stroke (width 0.2) (type default)) (layer "B.Cu") (net "Net-(J3-Pin_7)"))
 (gr_line (start 199 107) (end 197 107) (stroke (width 0.2) (type default)) (layer "B.Cu") (net "Net-(J3-Pin_8)"))
 (gr_line (start 199 107) (end 199 101) (stroke (width 0.2) (type default)) (layer "B.Cu") (net "Net-(J3-Pin_8)"))
 (gr_line (start 199.5 92.5) (end 202 92.5) (stroke (width 0.2) (type default)) (layer "B.Cu") (net "Net-(J3-Pin_6)"))
 (gr_line (start 199.5 109.5) (end 199.5 115) (stroke (width 0.2) (type default)) (layer "B.Cu") (net "Net-(J3-Pin_7)"))
 (gr_line (start 200.5 97.5) (end 200.5 109.5) (stroke (width 0.2) (type default)) (layer "B.Cu") (net "Net-(J3-Pin_7)"))
 (gr_line (start 200.5 109.5) (end 199.5 109.5) (stroke (width 0.2) (type default)) (layer "B.Cu") (net "Net-(J3-Pin_7)"))
 (gr_line (start 202 76.5) (end 202 82) (stroke (width 0.2) (type default)) (layer "B.Cu") (net "Net-(J3-Pin_9)"))
 (gr_line (start 202 82) (end 194.5 82) (stroke (width 0.2) (type default)) (layer "B.Cu") (net "Net-(J3-Pin_9)"))
 (gr_line (start 202 92.5) (end 202 114.97) (stroke (width 0.2) (type default)) (layer "B.Cu") (net "Net-(J3-Pin_6)"))
 (gr_line (start 211.5 82.5) (end 211.5 71.5) (stroke (width 0.2) (type default)) (layer "B.Cu") (net "Net-(J3-Pin_8)"))
 (gr_line (start 211.5 82.5) (end 211.5 86.5) (stroke (width 0.2) (type default)) (layer "B.Cu") (net "Net-(J3-Pin_8)"))
 (gr_line (start 211.5 86.5) (end 196.5 86.5) (stroke (width 0.2) (type default)) (layer "B.Cu") (net "Net-(J3-Pin_8)"))
 (gr_line (start 215.42 89) (end 197.5 89) (stroke (width 0.2) (type default)) (layer "B.Cu") (net "Net-(J3-Pin_7)"))
 (gr_line (start 215.42 92.5) (end 215.42 89) (stroke (width 0.2) (type default)) (layer "B.Cu") (net "Net-(J3-Pin_7)"))
 (gr_line (start 220.5 66.5) (end 220.5 71.5) (stroke (width 0.2) (type default)) (layer "B.Cu") (net "Net-(J3-Pin_8)"))
 (gr_line (start 220.5 71.5) (end 211.5 71.5) (stroke (width 0.2) (type default)) (layer "B.Cu") (net "Net-(J3-Pin_8)"))
 (gr_rect (start 164 63) (end 234 118) (stroke (width 0.05) (type default)) (fill no) (layer "Edge.Cuts"))
 (segment (start 230 64) (end 230 90) (width 0.2) (layer "F.Cu") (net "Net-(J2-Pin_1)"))
 (segment (start 182.78 64.72) (end 183.5 64) (width 0.2) (layer "F.Cu") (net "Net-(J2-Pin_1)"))
 (segment (start 183.5 64) (end 230 64) (width 0.2) (layer "F.Cu") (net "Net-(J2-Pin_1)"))
 (segment (start 182.78 66.71) (end 182.78 64.72) (width 0.2) (layer "F.Cu") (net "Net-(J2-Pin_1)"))
 (segment (start 230 117.35) (end 230 96) (width 0.2) (layer "F.Cu") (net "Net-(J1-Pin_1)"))
 (segment (start 187.86 116.01) (end 189.2 117.35) (width 0.2) (layer "F.Cu") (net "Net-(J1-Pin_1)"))
 (segment (start 187.86 114.96) (end 187.86 116.01) (width 0.2) (layer "F.Cu") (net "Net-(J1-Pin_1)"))
 (segment (start 189.2 117.35) (end 230 117.35) (width 0.2) (layer "F.Cu") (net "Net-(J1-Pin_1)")))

